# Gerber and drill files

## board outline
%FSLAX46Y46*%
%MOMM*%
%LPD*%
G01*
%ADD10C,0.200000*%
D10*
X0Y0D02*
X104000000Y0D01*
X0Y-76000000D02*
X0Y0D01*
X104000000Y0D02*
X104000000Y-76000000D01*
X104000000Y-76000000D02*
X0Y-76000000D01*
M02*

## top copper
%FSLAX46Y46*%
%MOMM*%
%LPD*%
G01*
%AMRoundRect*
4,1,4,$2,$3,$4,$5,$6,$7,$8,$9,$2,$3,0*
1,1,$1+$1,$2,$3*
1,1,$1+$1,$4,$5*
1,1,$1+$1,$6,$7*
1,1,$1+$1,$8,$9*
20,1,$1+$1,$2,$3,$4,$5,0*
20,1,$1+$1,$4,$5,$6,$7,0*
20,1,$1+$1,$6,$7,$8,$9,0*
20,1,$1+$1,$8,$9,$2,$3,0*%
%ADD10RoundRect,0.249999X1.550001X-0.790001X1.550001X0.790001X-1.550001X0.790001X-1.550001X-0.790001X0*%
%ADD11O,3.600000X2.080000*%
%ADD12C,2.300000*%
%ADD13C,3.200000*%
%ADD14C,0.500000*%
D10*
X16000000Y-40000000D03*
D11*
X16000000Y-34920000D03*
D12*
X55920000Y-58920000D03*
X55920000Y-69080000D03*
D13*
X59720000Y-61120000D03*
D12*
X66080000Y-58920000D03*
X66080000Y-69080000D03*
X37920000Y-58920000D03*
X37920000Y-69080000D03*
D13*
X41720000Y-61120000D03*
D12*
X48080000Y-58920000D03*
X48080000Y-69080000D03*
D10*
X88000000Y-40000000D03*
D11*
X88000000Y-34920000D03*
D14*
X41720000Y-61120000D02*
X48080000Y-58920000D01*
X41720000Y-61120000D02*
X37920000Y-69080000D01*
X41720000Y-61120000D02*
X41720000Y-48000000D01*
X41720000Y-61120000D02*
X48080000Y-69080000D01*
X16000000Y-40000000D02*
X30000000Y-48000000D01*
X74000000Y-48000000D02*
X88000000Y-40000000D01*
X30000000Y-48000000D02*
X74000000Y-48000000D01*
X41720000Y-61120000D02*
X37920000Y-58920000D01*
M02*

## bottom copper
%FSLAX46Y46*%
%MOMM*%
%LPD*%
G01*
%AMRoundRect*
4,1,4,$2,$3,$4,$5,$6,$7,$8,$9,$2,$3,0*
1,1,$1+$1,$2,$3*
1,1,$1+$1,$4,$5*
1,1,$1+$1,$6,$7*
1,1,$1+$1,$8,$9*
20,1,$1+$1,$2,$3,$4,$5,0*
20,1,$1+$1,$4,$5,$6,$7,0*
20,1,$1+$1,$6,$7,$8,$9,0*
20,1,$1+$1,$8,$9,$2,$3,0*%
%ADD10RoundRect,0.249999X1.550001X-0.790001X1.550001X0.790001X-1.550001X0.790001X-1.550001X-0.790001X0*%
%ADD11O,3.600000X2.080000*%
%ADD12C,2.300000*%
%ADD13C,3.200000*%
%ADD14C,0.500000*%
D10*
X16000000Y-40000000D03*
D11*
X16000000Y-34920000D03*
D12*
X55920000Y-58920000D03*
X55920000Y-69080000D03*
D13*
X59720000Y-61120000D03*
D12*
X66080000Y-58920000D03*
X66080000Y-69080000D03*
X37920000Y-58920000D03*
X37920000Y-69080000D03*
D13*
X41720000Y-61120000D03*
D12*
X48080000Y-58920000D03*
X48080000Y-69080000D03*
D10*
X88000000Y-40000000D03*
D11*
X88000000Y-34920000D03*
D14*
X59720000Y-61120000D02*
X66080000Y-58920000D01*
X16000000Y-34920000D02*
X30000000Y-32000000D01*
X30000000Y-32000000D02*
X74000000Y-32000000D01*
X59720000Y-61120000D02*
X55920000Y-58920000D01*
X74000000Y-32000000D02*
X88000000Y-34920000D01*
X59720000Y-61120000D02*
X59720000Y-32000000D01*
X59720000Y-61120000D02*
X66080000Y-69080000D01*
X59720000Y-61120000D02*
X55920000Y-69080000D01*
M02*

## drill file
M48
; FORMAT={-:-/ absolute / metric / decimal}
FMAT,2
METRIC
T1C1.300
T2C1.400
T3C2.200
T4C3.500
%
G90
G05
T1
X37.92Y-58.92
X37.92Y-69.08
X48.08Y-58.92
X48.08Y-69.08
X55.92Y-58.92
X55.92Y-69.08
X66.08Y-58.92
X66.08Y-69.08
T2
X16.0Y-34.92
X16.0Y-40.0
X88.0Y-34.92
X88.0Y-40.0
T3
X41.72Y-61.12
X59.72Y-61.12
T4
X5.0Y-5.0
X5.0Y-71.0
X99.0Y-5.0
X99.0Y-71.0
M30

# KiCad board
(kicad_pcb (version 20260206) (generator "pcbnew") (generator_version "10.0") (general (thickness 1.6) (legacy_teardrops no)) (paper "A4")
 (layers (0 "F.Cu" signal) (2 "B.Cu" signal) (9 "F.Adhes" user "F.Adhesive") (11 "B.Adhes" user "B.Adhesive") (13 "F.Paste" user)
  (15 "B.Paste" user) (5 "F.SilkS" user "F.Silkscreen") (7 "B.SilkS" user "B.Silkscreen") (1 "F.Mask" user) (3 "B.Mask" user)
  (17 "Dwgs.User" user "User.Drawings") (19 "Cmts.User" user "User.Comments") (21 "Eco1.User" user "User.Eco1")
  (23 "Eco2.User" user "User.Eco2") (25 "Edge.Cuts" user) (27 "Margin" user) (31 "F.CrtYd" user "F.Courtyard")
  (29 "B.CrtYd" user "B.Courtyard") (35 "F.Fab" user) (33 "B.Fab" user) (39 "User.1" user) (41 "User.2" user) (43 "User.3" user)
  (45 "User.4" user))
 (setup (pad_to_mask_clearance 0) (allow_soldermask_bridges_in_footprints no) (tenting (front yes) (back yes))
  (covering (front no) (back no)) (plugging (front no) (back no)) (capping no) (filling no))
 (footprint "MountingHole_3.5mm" (layer "F.Cu") (at 99 71)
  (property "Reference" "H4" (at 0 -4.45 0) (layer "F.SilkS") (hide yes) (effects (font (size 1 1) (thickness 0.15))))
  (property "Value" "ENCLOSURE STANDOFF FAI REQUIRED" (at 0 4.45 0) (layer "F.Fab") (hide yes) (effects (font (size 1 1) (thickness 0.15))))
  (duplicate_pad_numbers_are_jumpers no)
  (pad "" np_thru_hole circle (at 0 0) (size 3.5 3.5) (drill 3.5) (layers "*.Cu")))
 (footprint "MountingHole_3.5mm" (layer "F.Cu") (at 5 71)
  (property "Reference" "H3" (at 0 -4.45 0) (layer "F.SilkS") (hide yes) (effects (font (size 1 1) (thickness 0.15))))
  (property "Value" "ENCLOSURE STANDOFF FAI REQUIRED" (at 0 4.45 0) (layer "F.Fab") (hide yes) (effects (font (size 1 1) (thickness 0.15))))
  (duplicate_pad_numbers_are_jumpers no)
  (pad "" np_thru_hole circle (at 0 0) (size 3.5 3.5) (drill 3.5) (layers "*.Cu")))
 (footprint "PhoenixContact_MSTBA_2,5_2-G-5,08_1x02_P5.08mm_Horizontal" (layer "F.Cu") (at 16 40 90)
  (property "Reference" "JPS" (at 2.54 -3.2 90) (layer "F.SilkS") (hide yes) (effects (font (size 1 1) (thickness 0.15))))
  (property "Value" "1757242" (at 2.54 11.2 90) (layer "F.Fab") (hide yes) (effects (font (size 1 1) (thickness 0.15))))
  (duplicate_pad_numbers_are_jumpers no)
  (pad "1" thru_hole roundrect (at 0 0 90) (size 2.08 3.6) (drill 1.4) (layers "*.Cu") (remove_unused_layers no) (roundrect_rratio 0.120192)
   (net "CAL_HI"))
  (pad "2" thru_hole oval (at 5.08 0 90) (size 2.08 3.6) (drill 1.4) (layers "*.Cu") (remove_unused_layers no) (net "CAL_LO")))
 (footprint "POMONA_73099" (layer "F.Cu") (at 61 64)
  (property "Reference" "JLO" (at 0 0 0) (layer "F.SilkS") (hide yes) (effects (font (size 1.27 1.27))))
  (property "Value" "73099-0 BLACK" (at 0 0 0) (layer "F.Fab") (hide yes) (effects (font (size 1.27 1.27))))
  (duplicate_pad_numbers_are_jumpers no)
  (pad "1" thru_hole circle (at -5.08 -5.08) (size 2.3 2.3) (drill 1.3) (layers "*.Cu") (remove_unused_layers no) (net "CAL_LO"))
  (pad "1" thru_hole circle (at -5.08 5.08) (size 2.3 2.3) (drill 1.3) (layers "*.Cu") (remove_unused_layers no) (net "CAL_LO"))
  (pad "1" thru_hole circle (at -1.28 -2.88) (size 3.2 3.2) (drill 2.2) (layers "*.Cu") (remove_unused_layers no) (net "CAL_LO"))
  (pad "1" thru_hole circle (at 5.08 -5.08) (size 2.3 2.3) (drill 1.3) (layers "*.Cu") (remove_unused_layers no) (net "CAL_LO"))
  (pad "1" thru_hole circle (at 5.08 5.08) (size 2.3 2.3) (drill 1.3) (layers "*.Cu") (remove_unused_layers no) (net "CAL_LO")))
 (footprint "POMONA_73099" (layer "F.Cu") (at 43 64)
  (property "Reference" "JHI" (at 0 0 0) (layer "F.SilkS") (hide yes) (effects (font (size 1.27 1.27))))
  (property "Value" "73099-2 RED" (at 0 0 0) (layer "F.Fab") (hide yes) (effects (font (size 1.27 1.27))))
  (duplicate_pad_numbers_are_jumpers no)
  (pad "1" thru_hole circle (at -5.08 -5.08) (size 2.3 2.3) (drill 1.3) (layers "*.Cu") (remove_unused_layers no) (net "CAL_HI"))
  (pad "1" thru_hole circle (at -5.08 5.08) (size 2.3 2.3) (drill 1.3) (layers "*.Cu") (remove_unused_layers no) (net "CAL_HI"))
  (pad "1" thru_hole circle (at -1.28 -2.88) (size 3.2 3.2) (drill 2.2) (layers "*.Cu") (remove_unused_layers no) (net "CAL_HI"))
  (pad "1" thru_hole circle (at 5.08 -5.08) (size 2.3 2.3) (drill 1.3) (layers "*.Cu") (remove_unused_layers no) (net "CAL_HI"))
  (pad "1" thru_hole circle (at 5.08 5.08) (size 2.3 2.3) (drill 1.3) (layers "*.Cu") (remove_unused_layers no) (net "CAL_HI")))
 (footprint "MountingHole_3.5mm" (layer "F.Cu") (at 5 5)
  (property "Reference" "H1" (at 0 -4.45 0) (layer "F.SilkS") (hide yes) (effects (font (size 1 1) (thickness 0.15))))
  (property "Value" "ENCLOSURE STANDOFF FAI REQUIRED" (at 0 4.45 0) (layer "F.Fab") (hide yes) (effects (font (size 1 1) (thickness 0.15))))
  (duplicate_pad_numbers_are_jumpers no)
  (pad "" np_thru_hole circle (at 0 0) (size 3.5 3.5) (drill 3.5) (layers "*.Cu")))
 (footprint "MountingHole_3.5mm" (layer "F.Cu") (at 99 5)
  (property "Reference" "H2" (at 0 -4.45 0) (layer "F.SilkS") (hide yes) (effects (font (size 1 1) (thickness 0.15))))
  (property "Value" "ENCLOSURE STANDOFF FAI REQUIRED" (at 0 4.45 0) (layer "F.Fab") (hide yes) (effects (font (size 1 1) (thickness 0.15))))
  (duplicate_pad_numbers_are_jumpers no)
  (pad "" np_thru_hole circle (at 0 0) (size 3.5 3.5) (drill 3.5) (layers "*.Cu")))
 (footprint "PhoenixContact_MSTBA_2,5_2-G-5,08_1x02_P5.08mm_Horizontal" (layer "F.Cu") (at 88 40 90)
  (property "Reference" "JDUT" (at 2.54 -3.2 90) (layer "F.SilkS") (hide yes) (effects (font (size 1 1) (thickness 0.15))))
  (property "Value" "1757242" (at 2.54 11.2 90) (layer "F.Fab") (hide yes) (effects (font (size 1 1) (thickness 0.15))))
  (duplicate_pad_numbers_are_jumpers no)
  (pad "1" thru_hole roundrect (at 0 0 90) (size 2.08 3.6) (drill 1.4) (layers "*.Cu") (remove_unused_layers no) (roundrect_rratio 0.120192)
   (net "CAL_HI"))
  (pad "2" thru_hole oval (at 5.08 0 90) (size 2.08 3.6) (drill 1.4) (layers "*.Cu") (remove_unused_layers no) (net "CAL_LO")))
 (gr_line (start 0 0) (end 104 0) (stroke (width 0.2) (type default)) (layer "Edge.Cuts"))
 (gr_line (start 0 76) (end 0 0) (stroke (width 0.2) (type default)) (layer "Edge.Cuts"))
 (gr_line (start 104 0) (end 104 76) (stroke (width 0.2) (type default)) (layer "Edge.Cuts"))
 (gr_line (start 104 76) (end 0 76) (stroke (width 0.2) (type default)) (layer "Edge.Cuts"))
 (segment (start 41.72 61.12) (end 48.08 58.92) (width 0.5) (layer "F.Cu") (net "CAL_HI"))
 (segment (start 41.72 61.12) (end 37.92 69.08) (width 0.5) (layer "F.Cu") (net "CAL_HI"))
 (segment (start 41.72 61.12) (end 41.72 48) (width 0.5) (layer "F.Cu") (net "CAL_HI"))
 (segment (start 41.72 61.12) (end 48.08 69.08) (width 0.5) (layer "F.Cu") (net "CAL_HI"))
 (segment (start 16 40) (end 30 48) (width 0.5) (layer "F.Cu") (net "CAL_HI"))
 (segment (start 74 48) (end 88 40) (width 0.5) (layer "F.Cu") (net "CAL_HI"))
 (segment (start 30 48) (end 74 48) (width 0.5) (layer "F.Cu") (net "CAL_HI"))
 (segment (start 41.72 61.12) (end 37.92 58.92) (width 0.5) (layer "F.Cu") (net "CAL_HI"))
 (segment (start 59.72 61.12) (end 66.08 58.92) (width 0.5) (layer "B.Cu") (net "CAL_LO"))
 (segment (start 16 34.92) (end 30 32) (width 0.5) (layer "B.Cu") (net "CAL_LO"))
 (segment (start 30 32) (end 74 32) (width 0.5) (layer "B.Cu") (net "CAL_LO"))
 (segment (start 59.72 61.12) (end 55.92 58.92) (width 0.5) (layer "B.Cu") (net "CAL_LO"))
 (segment (start 74 32) (end 88 34.92) (width 0.5) (layer "B.Cu") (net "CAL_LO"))
 (segment (start 59.72 61.12) (end 59.72 32) (width 0.5) (layer "B.Cu") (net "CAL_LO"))
 (segment (start 59.72 61.12) (end 66.08 69.08) (width 0.5) (layer "B.Cu") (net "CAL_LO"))
 (segment (start 59.72 61.12) (end 55.92 69.08) (width 0.5) (layer "B.Cu") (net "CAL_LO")))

